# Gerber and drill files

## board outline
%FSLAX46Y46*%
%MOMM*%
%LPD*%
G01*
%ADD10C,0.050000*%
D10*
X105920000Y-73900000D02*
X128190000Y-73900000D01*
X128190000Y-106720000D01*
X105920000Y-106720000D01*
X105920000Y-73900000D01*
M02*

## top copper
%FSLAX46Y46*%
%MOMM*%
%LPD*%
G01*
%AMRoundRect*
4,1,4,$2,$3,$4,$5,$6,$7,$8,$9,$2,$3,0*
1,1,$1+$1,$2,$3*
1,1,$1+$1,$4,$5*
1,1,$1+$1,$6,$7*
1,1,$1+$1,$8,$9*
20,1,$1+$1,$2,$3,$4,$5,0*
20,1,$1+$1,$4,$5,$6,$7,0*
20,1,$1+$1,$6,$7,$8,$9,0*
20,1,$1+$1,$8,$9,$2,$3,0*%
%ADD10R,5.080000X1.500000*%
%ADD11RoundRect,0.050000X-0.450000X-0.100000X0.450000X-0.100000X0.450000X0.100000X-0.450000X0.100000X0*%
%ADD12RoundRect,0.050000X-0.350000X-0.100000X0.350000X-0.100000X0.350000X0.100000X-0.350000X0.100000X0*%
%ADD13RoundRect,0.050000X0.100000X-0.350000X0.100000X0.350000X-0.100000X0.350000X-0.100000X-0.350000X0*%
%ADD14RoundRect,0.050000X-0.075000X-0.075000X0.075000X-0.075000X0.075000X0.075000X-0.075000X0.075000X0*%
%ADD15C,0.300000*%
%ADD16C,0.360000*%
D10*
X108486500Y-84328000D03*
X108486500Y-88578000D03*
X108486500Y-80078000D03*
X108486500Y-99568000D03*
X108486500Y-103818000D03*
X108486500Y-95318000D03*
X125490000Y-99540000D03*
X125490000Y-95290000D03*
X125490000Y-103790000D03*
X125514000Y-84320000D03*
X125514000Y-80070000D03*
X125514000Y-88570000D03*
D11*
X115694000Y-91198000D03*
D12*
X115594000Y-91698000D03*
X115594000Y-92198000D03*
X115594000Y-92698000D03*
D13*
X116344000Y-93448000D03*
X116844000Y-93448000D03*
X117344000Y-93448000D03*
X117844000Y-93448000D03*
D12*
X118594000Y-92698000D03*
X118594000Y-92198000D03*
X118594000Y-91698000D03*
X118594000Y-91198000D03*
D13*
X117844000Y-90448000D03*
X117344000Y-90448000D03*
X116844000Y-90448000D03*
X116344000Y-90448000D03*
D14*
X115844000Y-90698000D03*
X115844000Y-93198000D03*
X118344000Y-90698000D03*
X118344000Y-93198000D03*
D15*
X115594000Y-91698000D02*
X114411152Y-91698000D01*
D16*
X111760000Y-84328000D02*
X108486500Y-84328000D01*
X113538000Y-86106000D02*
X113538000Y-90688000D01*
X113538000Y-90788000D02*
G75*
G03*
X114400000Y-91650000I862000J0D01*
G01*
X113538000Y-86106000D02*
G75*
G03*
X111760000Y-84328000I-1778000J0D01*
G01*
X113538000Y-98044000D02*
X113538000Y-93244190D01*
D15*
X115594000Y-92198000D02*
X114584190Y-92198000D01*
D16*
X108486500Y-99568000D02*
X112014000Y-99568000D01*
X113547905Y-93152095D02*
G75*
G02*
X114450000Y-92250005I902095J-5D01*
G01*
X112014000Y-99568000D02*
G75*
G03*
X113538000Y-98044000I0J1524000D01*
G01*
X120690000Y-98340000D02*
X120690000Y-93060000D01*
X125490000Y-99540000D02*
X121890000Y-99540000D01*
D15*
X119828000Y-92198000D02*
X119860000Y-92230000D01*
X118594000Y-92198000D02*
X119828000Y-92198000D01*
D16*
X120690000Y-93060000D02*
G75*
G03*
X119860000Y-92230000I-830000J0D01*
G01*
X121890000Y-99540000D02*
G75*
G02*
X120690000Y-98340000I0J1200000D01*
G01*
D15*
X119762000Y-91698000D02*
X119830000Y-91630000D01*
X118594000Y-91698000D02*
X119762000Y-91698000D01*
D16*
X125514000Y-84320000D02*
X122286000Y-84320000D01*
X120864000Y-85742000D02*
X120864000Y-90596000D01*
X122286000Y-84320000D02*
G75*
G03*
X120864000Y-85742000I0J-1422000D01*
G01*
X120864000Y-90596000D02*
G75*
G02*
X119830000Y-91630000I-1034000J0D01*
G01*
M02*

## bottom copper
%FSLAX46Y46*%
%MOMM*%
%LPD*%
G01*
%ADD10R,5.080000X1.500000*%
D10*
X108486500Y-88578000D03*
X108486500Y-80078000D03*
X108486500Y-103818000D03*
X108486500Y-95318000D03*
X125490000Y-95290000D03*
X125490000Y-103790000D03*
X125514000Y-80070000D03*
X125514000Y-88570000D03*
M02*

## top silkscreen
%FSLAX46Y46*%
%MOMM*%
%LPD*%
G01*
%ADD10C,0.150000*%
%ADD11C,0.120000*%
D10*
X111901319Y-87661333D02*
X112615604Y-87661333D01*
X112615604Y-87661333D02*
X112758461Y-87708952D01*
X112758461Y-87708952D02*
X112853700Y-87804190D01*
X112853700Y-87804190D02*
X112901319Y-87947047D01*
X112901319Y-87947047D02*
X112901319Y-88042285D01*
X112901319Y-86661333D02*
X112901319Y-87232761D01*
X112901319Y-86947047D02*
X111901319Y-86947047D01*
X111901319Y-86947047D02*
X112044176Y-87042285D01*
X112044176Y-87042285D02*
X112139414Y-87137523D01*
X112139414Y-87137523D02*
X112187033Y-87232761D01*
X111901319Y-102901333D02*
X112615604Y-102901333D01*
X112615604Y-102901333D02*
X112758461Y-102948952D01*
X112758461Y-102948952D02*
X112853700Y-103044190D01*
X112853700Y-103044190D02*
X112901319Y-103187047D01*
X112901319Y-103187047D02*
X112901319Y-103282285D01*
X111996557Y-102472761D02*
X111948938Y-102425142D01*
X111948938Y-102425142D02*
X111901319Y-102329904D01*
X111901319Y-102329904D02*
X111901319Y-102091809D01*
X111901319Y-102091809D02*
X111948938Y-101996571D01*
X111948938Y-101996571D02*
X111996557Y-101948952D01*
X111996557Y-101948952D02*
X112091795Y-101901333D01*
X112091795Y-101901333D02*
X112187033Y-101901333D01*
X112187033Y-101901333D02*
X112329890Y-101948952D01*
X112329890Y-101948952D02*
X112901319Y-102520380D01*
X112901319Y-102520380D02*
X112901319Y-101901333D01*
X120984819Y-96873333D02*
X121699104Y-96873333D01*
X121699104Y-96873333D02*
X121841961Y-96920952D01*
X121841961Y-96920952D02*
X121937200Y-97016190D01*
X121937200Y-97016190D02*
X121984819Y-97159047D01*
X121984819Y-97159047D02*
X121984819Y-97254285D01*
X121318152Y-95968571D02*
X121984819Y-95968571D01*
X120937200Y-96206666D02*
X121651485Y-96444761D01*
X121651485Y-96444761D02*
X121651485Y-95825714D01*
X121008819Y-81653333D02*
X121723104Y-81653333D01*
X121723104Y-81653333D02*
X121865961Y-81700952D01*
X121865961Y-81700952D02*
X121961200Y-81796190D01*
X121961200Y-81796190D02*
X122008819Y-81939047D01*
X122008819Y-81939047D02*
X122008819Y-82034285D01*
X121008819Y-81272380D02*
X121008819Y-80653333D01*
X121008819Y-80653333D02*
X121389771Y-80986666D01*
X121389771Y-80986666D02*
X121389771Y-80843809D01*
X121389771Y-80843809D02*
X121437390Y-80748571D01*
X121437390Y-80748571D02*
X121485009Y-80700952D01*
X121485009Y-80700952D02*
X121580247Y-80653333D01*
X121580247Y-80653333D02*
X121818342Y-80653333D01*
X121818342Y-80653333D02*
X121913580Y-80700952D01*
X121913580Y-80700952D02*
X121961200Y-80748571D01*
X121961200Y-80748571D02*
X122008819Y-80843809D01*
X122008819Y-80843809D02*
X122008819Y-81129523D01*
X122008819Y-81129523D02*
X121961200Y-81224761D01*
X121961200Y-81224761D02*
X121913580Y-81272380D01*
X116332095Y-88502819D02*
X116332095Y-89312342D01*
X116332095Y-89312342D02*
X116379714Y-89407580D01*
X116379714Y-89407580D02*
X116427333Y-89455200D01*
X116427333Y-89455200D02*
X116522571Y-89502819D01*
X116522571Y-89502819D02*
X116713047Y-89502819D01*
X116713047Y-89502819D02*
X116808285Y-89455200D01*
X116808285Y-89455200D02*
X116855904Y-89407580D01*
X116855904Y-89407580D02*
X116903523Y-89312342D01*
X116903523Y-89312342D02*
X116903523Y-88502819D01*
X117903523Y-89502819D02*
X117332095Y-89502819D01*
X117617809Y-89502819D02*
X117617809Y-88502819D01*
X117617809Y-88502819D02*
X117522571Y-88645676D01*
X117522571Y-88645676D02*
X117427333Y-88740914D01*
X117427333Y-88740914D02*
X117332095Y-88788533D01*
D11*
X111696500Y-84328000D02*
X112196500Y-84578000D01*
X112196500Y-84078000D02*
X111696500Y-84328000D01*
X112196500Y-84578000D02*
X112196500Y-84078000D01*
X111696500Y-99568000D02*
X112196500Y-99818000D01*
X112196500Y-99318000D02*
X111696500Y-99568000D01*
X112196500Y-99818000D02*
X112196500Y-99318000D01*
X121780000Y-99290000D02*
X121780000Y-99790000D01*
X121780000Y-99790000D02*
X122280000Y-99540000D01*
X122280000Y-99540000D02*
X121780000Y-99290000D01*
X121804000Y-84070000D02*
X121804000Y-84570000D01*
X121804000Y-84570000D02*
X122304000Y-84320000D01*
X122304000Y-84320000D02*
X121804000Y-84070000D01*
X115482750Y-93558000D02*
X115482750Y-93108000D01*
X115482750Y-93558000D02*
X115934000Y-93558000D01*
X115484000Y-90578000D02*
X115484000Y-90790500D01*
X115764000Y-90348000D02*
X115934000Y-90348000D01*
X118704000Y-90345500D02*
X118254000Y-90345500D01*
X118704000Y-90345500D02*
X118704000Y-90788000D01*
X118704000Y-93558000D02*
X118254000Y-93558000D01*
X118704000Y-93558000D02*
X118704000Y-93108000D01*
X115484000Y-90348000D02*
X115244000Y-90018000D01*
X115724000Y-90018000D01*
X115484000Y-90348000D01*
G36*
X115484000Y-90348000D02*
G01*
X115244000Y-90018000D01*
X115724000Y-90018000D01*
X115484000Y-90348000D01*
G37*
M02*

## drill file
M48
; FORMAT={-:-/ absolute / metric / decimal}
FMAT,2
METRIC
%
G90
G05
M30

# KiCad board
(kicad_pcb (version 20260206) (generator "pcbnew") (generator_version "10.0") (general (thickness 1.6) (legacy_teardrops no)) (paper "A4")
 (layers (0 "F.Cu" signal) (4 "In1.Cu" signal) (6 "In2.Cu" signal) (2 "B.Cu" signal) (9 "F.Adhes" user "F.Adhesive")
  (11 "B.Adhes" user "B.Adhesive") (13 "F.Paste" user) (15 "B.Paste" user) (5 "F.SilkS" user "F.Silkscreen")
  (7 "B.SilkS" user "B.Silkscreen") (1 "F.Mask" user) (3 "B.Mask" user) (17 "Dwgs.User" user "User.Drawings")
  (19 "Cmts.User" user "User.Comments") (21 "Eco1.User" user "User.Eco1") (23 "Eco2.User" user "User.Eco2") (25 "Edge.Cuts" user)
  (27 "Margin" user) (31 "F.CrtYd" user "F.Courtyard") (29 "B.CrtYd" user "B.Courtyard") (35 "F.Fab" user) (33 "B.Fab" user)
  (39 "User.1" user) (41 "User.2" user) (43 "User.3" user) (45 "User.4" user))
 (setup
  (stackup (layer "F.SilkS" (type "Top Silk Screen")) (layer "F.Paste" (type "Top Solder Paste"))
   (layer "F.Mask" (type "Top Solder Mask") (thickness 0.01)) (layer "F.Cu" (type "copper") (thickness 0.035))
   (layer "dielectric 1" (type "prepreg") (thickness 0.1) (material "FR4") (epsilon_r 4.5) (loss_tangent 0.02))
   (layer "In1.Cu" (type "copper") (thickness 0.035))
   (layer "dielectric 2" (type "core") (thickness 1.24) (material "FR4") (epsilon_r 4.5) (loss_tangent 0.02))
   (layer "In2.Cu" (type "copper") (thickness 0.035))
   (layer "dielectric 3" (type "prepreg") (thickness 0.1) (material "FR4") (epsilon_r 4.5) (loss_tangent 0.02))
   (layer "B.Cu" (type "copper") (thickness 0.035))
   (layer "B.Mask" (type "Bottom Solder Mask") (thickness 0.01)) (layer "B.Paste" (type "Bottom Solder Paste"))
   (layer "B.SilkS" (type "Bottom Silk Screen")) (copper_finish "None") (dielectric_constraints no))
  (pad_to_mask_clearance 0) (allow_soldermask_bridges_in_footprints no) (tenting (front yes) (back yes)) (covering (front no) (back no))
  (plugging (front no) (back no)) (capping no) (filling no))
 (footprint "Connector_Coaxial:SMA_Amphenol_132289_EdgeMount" (layer "F.Cu") (at 108.4865 84.328 180)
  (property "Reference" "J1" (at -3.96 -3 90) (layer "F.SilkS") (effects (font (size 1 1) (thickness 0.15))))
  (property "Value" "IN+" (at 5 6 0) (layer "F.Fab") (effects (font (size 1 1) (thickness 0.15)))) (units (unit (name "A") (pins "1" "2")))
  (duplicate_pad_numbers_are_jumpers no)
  (fp_line (start -3.21 0) (end -3.71 -0.25) (stroke (width 0.12) (type solid)) (layer "F.SilkS"))
  (fp_line (start -3.71 0.25) (end -3.21 0) (stroke (width 0.12) (type solid)) (layer "F.SilkS"))
  (fp_line (start -3.71 -0.25) (end -3.71 0.25) (stroke (width 0.12) (type solid)) (layer "F.SilkS"))
  (pad "1" smd rect (at 0 0 270) (size 1.5 5.08) (layers "F.Cu" "F.Mask" "F.Paste") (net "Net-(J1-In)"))
  (pad "2" smd rect (at 0 -4.25 270) (size 1.5 5.08) (layers "F.Cu" "F.Mask" "F.Paste") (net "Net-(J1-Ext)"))
  (pad "2" smd rect (at 0 -4.25 270) (size 1.5 5.08) (layers "B.Cu" "B.Mask" "B.Paste") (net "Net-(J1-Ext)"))
  (pad "2" smd rect (at 0 4.25 270) (size 1.5 5.08) (layers "F.Cu" "F.Mask" "F.Paste") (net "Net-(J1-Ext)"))
  (pad "2" smd rect (at 0 4.25 270) (size 1.5 5.08) (layers "B.Cu" "B.Mask" "B.Paste") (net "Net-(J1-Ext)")))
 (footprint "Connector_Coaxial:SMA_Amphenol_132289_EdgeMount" (layer "F.Cu") (at 108.4865 99.568 180)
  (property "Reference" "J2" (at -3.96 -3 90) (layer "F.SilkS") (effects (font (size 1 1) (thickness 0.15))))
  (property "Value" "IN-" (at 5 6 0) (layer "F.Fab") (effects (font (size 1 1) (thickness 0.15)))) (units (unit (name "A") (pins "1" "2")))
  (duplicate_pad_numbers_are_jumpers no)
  (fp_line (start -3.21 0) (end -3.71 -0.25) (stroke (width 0.12) (type solid)) (layer "F.SilkS"))
  (fp_line (start -3.71 0.25) (end -3.21 0) (stroke (width 0.12) (type solid)) (layer "F.SilkS"))
  (fp_line (start -3.71 -0.25) (end -3.71 0.25) (stroke (width 0.12) (type solid)) (layer "F.SilkS"))
  (pad "1" smd rect (at 0 0 270) (size 1.5 5.08) (layers "F.Cu" "F.Mask" "F.Paste") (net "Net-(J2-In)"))
  (pad "2" smd rect (at 0 -4.25 270) (size 1.5 5.08) (layers "F.Cu" "F.Mask" "F.Paste") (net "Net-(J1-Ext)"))
  (pad "2" smd rect (at 0 -4.25 270) (size 1.5 5.08) (layers "B.Cu" "B.Mask" "B.Paste") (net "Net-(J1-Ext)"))
  (pad "2" smd rect (at 0 4.25 270) (size 1.5 5.08) (layers "F.Cu" "F.Mask" "F.Paste") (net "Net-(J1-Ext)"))
  (pad "2" smd rect (at 0 4.25 270) (size 1.5 5.08) (layers "B.Cu" "B.Mask" "B.Paste") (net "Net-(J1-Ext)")))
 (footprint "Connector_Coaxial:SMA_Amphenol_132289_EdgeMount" (layer "F.Cu") (at 125.49 99.54)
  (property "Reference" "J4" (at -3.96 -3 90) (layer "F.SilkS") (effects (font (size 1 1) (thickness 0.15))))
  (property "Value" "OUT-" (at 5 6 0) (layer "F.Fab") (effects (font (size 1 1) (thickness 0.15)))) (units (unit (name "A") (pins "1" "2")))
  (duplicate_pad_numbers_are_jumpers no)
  (fp_line (start -3.71 -0.25) (end -3.71 0.25) (stroke (width 0.12) (type solid)) (layer "F.SilkS"))
  (fp_line (start -3.71 0.25) (end -3.21 0) (stroke (width 0.12) (type solid)) (layer "F.SilkS"))
  (fp_line (start -3.21 0) (end -3.71 -0.25) (stroke (width 0.12) (type solid)) (layer "F.SilkS"))
  (pad "1" smd rect (at 0 0 90) (size 1.5 5.08) (layers "F.Cu" "F.Mask" "F.Paste") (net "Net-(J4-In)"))
  (pad "2" smd rect (at 0 -4.25 90) (size 1.5 5.08) (layers "F.Cu" "F.Mask" "F.Paste") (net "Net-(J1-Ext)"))
  (pad "2" smd rect (at 0 -4.25 90) (size 1.5 5.08) (layers "B.Cu" "B.Mask" "B.Paste") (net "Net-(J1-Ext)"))
  (pad "2" smd rect (at 0 4.25 90) (size 1.5 5.08) (layers "F.Cu" "F.Mask" "F.Paste") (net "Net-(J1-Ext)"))
  (pad "2" smd rect (at 0 4.25 90) (size 1.5 5.08) (layers "B.Cu" "B.Mask" "B.Paste") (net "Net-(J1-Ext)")))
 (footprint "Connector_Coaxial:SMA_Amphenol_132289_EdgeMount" (layer "F.Cu") (at 125.514 84.32)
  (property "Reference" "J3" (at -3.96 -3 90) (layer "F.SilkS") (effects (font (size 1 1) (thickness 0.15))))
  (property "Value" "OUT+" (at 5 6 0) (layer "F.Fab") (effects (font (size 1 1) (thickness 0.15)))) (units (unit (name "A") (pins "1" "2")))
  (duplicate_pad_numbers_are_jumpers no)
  (fp_line (start -3.71 -0.25) (end -3.71 0.25) (stroke (width 0.12) (type solid)) (layer "F.SilkS"))
  (fp_line (start -3.71 0.25) (end -3.21 0) (stroke (width 0.12) (type solid)) (layer "F.SilkS"))
  (fp_line (start -3.21 0) (end -3.71 -0.25) (stroke (width 0.12) (type solid)) (layer "F.SilkS"))
  (pad "1" smd rect (at 0 0 90) (size 1.5 5.08) (layers "F.Cu" "F.Mask" "F.Paste") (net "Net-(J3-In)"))
  (pad "2" smd rect (at 0 -4.25 90) (size 1.5 5.08) (layers "F.Cu" "F.Mask" "F.Paste") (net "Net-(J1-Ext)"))
  (pad "2" smd rect (at 0 -4.25 90) (size 1.5 5.08) (layers "B.Cu" "B.Mask" "B.Paste") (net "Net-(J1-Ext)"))
  (pad "2" smd rect (at 0 4.25 90) (size 1.5 5.08) (layers "F.Cu" "F.Mask" "F.Paste") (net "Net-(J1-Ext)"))
  (pad "2" smd rect (at 0 4.25 90) (size 1.5 5.08) (layers "B.Cu" "B.Mask" "B.Paste") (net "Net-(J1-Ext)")))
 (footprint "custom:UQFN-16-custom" (layer "F.Cu") (at 117.094 91.948)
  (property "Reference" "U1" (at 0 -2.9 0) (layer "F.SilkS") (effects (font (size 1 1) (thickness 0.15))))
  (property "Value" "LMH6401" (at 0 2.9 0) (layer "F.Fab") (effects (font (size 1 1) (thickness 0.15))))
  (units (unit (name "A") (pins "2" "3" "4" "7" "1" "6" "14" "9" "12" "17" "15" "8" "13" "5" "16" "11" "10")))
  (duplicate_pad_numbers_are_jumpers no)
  (fp_line (start -1.61125 1.61) (end -1.61125 1.16) (stroke (width 0.12) (type solid)) (layer "F.SilkS"))
  (fp_line (start -1.61125 1.61) (end -1.16 1.61) (stroke (width 0.12) (type solid)) (layer "F.SilkS"))
  (fp_line (start -1.61 -1.37) (end -1.61 -1.1575) (stroke (width 0.12) (type solid)) (layer "F.SilkS"))
  (fp_line (start -1.33 -1.6) (end -1.16 -1.6) (stroke (width 0.12) (type solid)) (layer "F.SilkS"))
  (fp_line (start 1.61 -1.6025) (end 1.16 -1.6025) (stroke (width 0.12) (type solid)) (layer "F.SilkS"))
  (fp_line (start 1.61 -1.6025) (end 1.61 -1.16) (stroke (width 0.12) (type solid)) (layer "F.SilkS"))
  (fp_line (start 1.61 1.61) (end 1.16 1.61) (stroke (width 0.12) (type solid)) (layer "F.SilkS"))
  (fp_line (start 1.61 1.61) (end 1.61 1.16) (stroke (width 0.12) (type solid)) (layer "F.SilkS"))
  (fp_poly
   (pts (xy -1.61 -1.6) (xy -1.85 -1.93) (xy -1.37 -1.93) (xy -1.61 -1.6)) (stroke (width 0.12) (type solid)) (fill yes) (layer "F.SilkS"))
  (pad "1" smd roundrect (at -1.4 -0.75) (size 1 0.3) (layers "F.Cu" "F.Mask" "F.Paste") (roundrect_rratio 0.1666666667)
   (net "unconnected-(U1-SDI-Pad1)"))
  (pad "2" smd roundrect (at -1.5 -0.25) (size 0.8 0.3) (layers "F.Cu" "F.Mask" "F.Paste") (roundrect_rratio 0.1666666667)
   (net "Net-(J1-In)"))
  (pad "3" smd roundrect (at -1.5 0.25) (size 0.8 0.3) (layers "F.Cu" "F.Mask" "F.Paste") (roundrect_rratio 0.1666666667)
   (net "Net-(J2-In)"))
  (pad "4" smd roundrect (at -1.5 0.75) (size 0.8 0.3) (layers "F.Cu" "F.Mask" "F.Paste") (roundrect_rratio 0.1666666667)
   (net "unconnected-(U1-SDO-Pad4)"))
  (pad "5" smd roundrect (at -0.75 1.5 90) (size 0.8 0.3) (layers "F.Cu" "F.Mask" "F.Paste") (roundrect_rratio 0.1666666667)
   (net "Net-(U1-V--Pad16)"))
  (pad "6" smd roundrect (at -0.25 1.5 90) (size 0.8 0.3) (layers "F.Cu" "F.Mask" "F.Paste") (roundrect_rratio 0.1666666667)
   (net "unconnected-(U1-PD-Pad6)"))
  (pad "7" smd roundrect (at 0.25 1.5 90) (size 0.8 0.3) (layers "F.Cu" "F.Mask" "F.Paste") (roundrect_rratio 0.1666666667)
   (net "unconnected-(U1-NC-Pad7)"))
  (pad "8" smd roundrect (at 0.75 1.5 90) (size 0.8 0.3) (layers "F.Cu" "F.Mask" "F.Paste") (roundrect_rratio 0.1666666667)
   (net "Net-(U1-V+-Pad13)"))
  (pad "9" smd roundrect (at 1.5 0.75) (size 0.8 0.3) (layers "F.Cu" "F.Mask" "F.Paste") (roundrect_rratio 0.1666666667)
   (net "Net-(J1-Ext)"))
  (pad "10" smd roundrect (at 1.5 0.25) (size 0.8 0.3) (layers "F.Cu" "F.Mask" "F.Paste") (roundrect_rratio 0.1666666667)
   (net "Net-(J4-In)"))
  (pad "11" smd roundrect (at 1.5 -0.25) (size 0.8 0.3) (layers "F.Cu" "F.Mask" "F.Paste") (roundrect_rratio 0.1666666667)
   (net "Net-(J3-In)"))
  (pad "12" smd roundrect (at 1.5 -0.75) (size 0.8 0.3) (layers "F.Cu" "F.Mask" "F.Paste") (roundrect_rratio 0.1666666667)
   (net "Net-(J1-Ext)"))
  (pad "13" smd roundrect (at 0.75 -1.5 90) (size 0.8 0.3) (layers "F.Cu" "F.Mask" "F.Paste") (roundrect_rratio 0.1666666667)
   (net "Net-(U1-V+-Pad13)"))
  (pad "14" smd roundrect (at 0.25 -1.5 90) (size 0.8 0.3) (layers "F.Cu" "F.Mask" "F.Paste") (roundrect_rratio 0.1666666667)
   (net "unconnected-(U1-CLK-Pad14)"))
  (pad "15" smd roundrect (at -0.25 -1.5 90) (size 0.8 0.3) (layers "F.Cu" "F.Mask" "F.Paste") (roundrect_rratio 0.1666666667)
   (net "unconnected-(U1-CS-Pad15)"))
  (pad "16" smd roundrect (at -0.75 -1.5 90) (size 0.8 0.3) (layers "F.Cu" "F.Mask" "F.Paste") (roundrect_rratio 0.1666666667)
   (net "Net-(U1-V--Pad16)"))
  (pad "17" smd roundrect (at -1.25 -1.25) (size 0.25 0.25) (layers "F.Cu" "F.Mask") (roundrect_rratio 0.2) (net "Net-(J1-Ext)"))
  (pad "17" smd roundrect (at -1.25 1.25) (size 0.25 0.25) (layers "F.Cu" "F.Mask") (roundrect_rratio 0.2) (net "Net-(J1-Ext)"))
  (pad "17" smd roundrect (at 1.25 -1.25) (size 0.25 0.25) (layers "F.Cu" "F.Mask") (roundrect_rratio 0.2) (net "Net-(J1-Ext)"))
  (pad "17" smd roundrect (at 1.25 1.25) (size 0.25 0.25) (layers "F.Cu" "F.Mask") (roundrect_rratio 0.2) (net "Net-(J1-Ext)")))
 (gr_rect (start 105.92 73.9) (end 128.19 106.72) (stroke (width 0.05) (type default)) (fill no) (layer "Edge.Cuts"))
 (segment (start 115.594 91.698) (end 114.411152 91.698) (width 0.3) (layer "F.Cu") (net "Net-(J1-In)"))
 (segment (start 111.76 84.328) (end 108.4865 84.328) (width 0.36) (layer "F.Cu") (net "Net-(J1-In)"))
 (segment (start 113.538 86.106) (end 113.538 90.688) (width 0.36) (layer "F.Cu") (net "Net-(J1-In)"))
 (arc (start 113.538 90.788) (mid 113.790474 91.397526) (end 114.4 91.65) (width 0.36) (layer "F.Cu") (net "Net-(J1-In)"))
 (arc (start 113.538 86.106) (mid 113.017236 84.848764) (end 111.76 84.328) (width 0.36) (layer "F.Cu") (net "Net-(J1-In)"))
 (segment (start 113.538 98.044) (end 113.538 93.24419) (width 0.36) (layer "F.Cu") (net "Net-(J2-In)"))
 (segment (start 115.594 92.198) (end 114.58419 92.198) (width 0.3) (layer "F.Cu") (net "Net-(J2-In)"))
 (segment (start 108.4865 99.568) (end 112.014 99.568) (width 0.36) (layer "F.Cu") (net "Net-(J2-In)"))
 (arc (start 113.547905 93.152095) (mid 113.812123 92.514218) (end 114.45 92.25) (width 0.36) (layer "F.Cu") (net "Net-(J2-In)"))
 (arc (start 112.014 99.568) (mid 113.091631 99.121631) (end 113.538 98.044) (width 0.36) (layer "F.Cu") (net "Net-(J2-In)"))
 (segment (start 120.69 98.34) (end 120.69 93.06) (width 0.36) (layer "F.Cu") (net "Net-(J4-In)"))
 (segment (start 125.49 99.54) (end 121.89 99.54) (width 0.36) (layer "F.Cu") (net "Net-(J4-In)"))
 (segment (start 119.828 92.198) (end 119.86 92.23) (width 0.3) (layer "F.Cu") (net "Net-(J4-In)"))
 (segment (start 118.594 92.198) (end 119.828 92.198) (width 0.3) (layer "F.Cu") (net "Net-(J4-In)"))
 (arc (start 120.69 93.06) (mid 120.446899 92.473101) (end 119.86 92.23) (width 0.36) (layer "F.Cu") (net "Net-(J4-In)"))
 (arc (start 121.89 99.54) (mid 121.041472 99.188528) (end 120.69 98.34) (width 0.36) (layer "F.Cu") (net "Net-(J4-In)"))
 (segment (start 119.762 91.698) (end 119.83 91.63) (width 0.3) (layer "F.Cu") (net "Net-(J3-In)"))
 (segment (start 118.594 91.698) (end 119.762 91.698) (width 0.3) (layer "F.Cu") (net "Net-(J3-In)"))
 (segment (start 125.514 84.32) (end 122.286 84.32) (width 0.36) (layer "F.Cu") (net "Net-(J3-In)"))
 (segment (start 120.864 85.742) (end 120.864 90.596) (width 0.36) (layer "F.Cu") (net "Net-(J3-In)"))
 (arc (start 122.286 84.32) (mid 121.280494 84.736494) (end 120.864 85.742) (width 0.36) (layer "F.Cu") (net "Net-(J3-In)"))
 (arc (start 120.864 90.596) (mid 120.561148 91.327148) (end 119.83 91.63) (width 0.36) (layer "F.Cu") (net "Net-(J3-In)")))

